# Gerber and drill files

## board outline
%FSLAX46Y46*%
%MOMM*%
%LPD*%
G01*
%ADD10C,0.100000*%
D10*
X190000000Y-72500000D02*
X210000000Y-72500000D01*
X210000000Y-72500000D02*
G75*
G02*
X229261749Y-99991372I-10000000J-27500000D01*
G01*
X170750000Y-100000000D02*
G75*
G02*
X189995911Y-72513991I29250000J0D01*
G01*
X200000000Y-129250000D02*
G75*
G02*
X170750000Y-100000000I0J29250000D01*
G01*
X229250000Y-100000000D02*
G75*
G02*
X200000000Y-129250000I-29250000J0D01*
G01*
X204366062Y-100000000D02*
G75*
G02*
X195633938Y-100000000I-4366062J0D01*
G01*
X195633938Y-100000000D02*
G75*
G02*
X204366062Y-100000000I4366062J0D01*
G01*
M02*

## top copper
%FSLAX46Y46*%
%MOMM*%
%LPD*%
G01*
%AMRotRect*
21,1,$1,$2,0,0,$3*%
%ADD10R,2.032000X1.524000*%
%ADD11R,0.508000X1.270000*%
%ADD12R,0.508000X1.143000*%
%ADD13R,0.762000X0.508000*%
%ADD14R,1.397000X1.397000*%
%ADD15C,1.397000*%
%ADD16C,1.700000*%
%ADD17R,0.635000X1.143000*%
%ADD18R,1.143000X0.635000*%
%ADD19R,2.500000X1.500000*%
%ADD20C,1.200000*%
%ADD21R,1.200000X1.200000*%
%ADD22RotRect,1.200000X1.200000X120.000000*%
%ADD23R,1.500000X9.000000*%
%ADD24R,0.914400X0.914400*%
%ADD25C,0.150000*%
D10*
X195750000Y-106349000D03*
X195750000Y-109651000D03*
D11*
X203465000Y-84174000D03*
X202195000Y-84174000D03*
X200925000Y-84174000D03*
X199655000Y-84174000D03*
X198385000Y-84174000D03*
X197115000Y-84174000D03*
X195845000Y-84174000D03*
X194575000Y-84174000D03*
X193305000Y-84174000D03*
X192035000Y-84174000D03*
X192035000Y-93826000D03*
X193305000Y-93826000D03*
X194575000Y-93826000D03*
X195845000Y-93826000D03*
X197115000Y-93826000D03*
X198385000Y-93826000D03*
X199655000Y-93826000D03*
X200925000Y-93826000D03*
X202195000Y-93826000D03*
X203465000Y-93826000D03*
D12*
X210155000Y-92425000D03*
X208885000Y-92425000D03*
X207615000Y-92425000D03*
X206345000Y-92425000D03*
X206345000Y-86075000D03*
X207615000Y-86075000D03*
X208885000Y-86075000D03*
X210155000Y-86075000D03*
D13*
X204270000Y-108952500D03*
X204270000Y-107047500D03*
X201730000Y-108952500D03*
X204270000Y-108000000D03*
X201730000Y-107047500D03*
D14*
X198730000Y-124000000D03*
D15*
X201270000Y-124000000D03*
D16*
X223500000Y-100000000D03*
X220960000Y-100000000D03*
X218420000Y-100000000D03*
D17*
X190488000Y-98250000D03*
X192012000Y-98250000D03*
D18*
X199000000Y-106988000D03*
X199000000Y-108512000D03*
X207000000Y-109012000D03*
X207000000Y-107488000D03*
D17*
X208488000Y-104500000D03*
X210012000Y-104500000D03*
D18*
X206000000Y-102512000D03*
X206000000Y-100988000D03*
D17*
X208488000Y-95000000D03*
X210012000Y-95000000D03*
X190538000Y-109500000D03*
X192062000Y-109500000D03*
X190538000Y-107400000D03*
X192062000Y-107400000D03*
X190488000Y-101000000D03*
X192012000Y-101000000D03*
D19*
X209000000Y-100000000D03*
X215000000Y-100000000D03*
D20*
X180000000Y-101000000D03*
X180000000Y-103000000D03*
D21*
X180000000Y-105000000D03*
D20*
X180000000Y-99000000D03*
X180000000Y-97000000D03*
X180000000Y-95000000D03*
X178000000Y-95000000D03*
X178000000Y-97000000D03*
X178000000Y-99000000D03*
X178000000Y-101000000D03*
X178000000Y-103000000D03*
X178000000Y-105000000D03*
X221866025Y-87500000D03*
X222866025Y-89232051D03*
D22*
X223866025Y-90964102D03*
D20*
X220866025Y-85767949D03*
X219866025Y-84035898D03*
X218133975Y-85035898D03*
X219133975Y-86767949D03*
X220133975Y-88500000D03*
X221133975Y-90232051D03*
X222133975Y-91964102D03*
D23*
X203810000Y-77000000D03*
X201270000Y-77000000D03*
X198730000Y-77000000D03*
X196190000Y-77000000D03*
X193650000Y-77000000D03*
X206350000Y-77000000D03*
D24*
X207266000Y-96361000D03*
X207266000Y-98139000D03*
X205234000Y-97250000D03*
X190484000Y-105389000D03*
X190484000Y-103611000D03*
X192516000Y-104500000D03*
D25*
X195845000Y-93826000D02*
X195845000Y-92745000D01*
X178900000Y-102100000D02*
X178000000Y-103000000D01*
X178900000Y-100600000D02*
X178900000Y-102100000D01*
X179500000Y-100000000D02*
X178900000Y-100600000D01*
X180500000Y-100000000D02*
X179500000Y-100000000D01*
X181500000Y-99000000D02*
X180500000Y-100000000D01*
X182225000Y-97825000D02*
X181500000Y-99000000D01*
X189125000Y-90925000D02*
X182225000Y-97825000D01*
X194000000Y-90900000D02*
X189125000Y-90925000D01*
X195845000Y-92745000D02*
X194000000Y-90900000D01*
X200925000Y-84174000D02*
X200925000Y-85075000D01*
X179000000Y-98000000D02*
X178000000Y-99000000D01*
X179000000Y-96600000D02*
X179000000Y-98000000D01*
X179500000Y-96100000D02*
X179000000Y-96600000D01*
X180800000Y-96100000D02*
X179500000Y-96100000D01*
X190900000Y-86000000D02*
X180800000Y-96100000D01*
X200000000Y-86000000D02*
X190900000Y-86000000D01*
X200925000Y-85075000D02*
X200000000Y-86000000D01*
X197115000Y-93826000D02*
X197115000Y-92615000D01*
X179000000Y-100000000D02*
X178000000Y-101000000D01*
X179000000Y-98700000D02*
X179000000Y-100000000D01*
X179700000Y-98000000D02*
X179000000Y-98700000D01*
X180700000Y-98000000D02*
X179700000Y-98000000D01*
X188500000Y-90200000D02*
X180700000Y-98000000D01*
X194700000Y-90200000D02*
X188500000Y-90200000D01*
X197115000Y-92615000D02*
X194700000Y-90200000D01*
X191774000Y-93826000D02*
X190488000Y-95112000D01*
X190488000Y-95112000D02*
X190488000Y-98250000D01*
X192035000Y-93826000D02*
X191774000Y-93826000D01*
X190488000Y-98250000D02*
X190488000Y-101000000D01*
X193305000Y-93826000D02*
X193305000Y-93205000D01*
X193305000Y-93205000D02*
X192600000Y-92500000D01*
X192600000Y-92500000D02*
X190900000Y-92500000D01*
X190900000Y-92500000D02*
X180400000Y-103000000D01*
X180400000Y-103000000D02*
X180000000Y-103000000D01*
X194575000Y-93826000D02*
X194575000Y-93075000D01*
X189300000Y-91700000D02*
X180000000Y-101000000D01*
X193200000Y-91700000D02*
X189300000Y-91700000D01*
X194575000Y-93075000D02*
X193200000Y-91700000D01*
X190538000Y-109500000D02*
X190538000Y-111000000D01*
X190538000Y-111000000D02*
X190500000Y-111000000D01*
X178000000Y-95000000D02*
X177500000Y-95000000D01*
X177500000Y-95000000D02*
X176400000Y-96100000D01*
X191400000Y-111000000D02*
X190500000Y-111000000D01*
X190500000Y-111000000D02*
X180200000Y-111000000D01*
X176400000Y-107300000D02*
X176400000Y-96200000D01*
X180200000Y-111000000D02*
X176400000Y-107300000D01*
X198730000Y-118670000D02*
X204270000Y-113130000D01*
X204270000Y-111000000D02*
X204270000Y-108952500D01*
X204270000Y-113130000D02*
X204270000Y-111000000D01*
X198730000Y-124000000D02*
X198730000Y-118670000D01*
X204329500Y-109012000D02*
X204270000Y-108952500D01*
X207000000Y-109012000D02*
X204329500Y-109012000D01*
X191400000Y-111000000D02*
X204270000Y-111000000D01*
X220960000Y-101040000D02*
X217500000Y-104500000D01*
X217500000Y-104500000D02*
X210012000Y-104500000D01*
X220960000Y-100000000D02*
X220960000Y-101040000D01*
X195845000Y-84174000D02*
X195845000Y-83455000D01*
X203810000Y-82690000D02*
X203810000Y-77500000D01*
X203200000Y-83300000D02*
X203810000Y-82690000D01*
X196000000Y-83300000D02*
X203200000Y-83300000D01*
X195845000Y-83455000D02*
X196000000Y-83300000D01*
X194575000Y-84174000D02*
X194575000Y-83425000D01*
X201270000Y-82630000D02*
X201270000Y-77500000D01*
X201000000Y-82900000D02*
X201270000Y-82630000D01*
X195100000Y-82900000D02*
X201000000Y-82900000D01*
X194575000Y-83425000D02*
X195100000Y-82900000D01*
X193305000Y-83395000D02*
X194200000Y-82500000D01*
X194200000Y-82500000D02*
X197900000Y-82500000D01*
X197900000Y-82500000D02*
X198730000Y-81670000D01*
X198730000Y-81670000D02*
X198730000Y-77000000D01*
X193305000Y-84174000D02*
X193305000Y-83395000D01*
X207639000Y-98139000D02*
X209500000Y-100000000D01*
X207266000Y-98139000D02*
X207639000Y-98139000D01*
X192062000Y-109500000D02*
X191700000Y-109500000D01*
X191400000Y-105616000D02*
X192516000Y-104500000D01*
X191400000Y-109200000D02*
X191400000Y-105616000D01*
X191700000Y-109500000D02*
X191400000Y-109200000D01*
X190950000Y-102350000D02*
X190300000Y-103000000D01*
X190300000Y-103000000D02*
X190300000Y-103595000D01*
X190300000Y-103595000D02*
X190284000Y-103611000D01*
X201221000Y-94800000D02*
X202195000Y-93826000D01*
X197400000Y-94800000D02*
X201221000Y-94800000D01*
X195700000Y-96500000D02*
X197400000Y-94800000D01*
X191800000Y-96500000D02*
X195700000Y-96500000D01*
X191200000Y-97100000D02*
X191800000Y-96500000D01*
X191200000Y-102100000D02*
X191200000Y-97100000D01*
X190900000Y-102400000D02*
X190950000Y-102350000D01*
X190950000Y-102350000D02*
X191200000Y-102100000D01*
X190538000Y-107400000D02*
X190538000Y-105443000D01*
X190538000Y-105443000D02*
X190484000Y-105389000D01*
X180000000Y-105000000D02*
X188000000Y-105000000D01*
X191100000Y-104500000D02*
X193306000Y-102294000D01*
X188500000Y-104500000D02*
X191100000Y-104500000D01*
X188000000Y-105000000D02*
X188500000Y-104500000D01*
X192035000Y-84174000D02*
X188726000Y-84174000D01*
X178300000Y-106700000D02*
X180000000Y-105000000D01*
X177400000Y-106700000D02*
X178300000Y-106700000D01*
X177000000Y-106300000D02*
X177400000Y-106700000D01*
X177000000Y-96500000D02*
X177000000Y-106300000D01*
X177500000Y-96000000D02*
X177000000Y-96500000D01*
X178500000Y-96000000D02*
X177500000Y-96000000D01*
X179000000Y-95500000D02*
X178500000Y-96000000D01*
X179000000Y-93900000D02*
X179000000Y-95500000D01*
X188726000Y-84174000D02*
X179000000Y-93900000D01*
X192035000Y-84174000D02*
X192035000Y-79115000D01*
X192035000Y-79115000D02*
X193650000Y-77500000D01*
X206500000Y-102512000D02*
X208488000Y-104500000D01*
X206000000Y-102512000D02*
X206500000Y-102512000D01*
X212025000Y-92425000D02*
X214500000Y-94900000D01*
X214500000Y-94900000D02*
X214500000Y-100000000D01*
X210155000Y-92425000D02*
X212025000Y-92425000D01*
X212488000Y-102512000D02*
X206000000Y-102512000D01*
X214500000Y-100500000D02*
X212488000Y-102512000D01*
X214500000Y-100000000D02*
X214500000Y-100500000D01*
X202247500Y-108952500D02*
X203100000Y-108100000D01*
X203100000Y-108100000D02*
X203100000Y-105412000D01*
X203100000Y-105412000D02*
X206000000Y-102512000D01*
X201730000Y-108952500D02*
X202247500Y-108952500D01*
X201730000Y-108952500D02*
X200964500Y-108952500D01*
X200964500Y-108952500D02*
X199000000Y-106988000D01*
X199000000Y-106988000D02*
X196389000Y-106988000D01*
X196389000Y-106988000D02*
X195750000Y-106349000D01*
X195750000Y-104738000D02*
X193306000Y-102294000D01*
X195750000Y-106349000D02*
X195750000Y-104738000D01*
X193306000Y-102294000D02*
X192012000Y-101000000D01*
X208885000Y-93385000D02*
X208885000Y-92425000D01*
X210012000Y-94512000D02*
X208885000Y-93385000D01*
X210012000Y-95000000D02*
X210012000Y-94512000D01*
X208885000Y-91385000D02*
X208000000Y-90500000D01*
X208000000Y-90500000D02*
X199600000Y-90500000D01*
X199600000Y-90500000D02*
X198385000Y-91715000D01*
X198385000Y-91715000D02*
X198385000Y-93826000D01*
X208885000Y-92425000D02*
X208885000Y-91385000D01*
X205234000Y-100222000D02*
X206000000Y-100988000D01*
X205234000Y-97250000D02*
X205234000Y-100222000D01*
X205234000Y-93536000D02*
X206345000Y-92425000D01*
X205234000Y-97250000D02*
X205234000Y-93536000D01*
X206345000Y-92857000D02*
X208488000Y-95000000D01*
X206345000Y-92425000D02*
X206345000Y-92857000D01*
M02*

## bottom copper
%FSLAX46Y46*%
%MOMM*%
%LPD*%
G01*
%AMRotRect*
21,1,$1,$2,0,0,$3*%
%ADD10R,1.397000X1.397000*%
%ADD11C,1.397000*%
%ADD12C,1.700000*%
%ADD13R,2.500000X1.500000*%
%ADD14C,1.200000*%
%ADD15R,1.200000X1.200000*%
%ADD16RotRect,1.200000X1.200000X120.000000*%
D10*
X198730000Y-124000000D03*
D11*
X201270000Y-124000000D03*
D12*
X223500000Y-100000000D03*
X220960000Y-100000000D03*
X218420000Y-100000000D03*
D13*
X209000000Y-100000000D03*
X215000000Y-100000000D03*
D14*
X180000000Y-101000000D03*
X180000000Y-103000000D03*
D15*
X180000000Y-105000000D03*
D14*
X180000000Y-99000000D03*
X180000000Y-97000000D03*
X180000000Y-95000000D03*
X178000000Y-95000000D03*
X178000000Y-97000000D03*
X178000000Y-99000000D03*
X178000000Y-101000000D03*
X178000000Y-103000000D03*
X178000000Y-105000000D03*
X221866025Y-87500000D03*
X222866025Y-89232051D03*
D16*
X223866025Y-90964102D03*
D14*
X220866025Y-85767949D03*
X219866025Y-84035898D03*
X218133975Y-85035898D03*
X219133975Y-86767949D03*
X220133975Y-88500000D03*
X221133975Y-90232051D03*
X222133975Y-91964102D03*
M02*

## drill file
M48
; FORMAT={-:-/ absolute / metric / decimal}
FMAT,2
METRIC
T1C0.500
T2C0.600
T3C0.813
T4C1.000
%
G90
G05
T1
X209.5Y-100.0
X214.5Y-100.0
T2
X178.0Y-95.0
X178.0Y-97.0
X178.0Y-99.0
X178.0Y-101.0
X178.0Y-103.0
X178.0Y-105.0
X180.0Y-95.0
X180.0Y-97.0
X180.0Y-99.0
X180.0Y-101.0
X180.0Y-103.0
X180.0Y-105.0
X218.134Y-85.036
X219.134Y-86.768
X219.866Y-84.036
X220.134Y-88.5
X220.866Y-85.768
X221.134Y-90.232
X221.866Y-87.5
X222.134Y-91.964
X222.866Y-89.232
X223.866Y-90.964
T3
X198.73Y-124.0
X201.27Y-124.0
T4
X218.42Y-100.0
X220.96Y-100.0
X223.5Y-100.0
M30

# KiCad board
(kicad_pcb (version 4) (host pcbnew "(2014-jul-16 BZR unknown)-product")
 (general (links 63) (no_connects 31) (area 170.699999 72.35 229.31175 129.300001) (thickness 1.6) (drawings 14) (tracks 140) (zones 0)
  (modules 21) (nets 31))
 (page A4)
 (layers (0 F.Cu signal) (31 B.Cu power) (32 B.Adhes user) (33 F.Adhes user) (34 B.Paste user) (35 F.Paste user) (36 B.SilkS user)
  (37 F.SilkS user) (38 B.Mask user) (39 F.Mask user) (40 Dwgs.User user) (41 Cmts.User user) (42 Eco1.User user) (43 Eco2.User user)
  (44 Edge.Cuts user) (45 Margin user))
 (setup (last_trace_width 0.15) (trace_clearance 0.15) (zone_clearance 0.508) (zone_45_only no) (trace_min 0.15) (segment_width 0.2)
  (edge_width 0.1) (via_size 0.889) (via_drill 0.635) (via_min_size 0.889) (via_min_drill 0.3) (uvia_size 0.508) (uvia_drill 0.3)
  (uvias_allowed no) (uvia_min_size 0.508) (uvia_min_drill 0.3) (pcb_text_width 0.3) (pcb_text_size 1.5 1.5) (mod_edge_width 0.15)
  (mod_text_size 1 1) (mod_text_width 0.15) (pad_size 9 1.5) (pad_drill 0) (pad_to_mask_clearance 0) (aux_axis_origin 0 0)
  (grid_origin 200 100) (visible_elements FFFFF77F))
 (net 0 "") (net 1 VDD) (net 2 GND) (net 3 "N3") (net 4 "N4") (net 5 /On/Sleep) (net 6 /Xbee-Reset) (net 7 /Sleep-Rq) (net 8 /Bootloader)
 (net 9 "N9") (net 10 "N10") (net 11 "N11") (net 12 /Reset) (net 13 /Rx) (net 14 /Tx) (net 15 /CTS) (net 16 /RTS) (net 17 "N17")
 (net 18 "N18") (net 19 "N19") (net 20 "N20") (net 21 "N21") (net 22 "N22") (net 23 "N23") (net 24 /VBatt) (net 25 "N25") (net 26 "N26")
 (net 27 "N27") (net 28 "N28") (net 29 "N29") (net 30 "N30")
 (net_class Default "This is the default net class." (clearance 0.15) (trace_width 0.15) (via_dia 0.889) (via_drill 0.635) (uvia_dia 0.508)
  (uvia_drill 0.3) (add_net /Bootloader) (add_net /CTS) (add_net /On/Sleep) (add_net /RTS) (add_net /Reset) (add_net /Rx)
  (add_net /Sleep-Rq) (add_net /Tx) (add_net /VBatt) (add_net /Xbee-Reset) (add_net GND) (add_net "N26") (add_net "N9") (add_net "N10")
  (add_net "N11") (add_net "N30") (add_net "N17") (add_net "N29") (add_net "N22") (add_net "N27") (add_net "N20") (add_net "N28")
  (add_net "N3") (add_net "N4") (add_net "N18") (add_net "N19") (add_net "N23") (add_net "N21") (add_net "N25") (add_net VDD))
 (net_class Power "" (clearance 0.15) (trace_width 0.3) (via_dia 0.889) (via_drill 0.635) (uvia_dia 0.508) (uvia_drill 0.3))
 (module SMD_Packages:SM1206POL (layer F.Cu) (at 195.75 108 270)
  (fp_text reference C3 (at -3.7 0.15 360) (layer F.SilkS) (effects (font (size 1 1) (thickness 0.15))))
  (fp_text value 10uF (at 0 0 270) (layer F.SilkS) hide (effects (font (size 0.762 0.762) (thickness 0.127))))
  (pad 1 smd rect (at -1.651 0 270) (size 1.524 2.032) (layers F.Cu F.Paste F.Mask) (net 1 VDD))
  (pad 2 smd rect (at 1.651 0 270) (size 1.524 2.032) (layers F.Cu F.Paste F.Mask) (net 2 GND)))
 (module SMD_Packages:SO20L (layer F.Cu) (at 197.75 89)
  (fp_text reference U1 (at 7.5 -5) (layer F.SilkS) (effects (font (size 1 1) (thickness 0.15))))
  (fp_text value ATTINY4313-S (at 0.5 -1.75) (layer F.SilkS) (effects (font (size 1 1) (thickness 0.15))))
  (pad 11 smd rect (at 5.715 -4.826) (size 0.508 1.27) (layers F.Cu F.Paste F.Mask) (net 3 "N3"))
  (pad 12 smd rect (at 4.445 -4.826) (size 0.508 1.27) (layers F.Cu F.Paste F.Mask) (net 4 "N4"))
  (pad 13 smd rect (at 3.175 -4.826) (size 0.508 1.27) (layers F.Cu F.Paste F.Mask) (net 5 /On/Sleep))
  (pad 14 smd rect (at 1.905 -4.826) (size 0.508 1.27) (layers F.Cu F.Paste F.Mask) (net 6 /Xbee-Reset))
  (pad 15 smd rect (at 0.635 -4.826) (size 0.508 1.27) (layers F.Cu F.Paste F.Mask) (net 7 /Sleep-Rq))
  (pad 16 smd rect (at -0.635 -4.826) (size 0.508 1.27) (layers F.Cu F.Paste F.Mask) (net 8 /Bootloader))
  (pad 17 smd rect (at -1.905 -4.826) (size 0.508 1.27) (layers F.Cu F.Paste F.Mask) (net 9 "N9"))
  (pad 18 smd rect (at -3.175 -4.826) (size 0.508 1.27) (layers F.Cu F.Paste F.Mask) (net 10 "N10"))
  (pad 19 smd rect (at -4.445 -4.826) (size 0.508 1.27) (layers F.Cu F.Paste F.Mask) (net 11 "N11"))
  (pad 20 smd rect (at -5.715 -4.826) (size 0.508 1.27) (layers F.Cu F.Paste F.Mask) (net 1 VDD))
  (pad 1 smd rect (at -5.715 4.826) (size 0.508 1.27) (layers F.Cu F.Paste F.Mask) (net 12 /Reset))
  (pad 2 smd rect (at -4.445 4.826) (size 0.508 1.27) (layers F.Cu F.Paste F.Mask) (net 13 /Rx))
  (pad 3 smd rect (at -3.175 4.826) (size 0.508 1.27) (layers F.Cu F.Paste F.Mask) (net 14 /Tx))
  (pad 4 smd rect (at -1.905 4.826) (size 0.508 1.27) (layers F.Cu F.Paste F.Mask) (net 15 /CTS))
  (pad 5 smd rect (at -0.635 4.826) (size 0.508 1.27) (layers F.Cu F.Paste F.Mask) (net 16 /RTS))
  (pad 6 smd rect (at 0.635 4.826) (size 0.508 1.27) (layers F.Cu F.Paste F.Mask) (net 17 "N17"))
  (pad 7 smd rect (at 1.905 4.826) (size 0.508 1.27) (layers F.Cu F.Paste F.Mask) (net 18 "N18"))
  (pad 8 smd rect (at 3.175 4.826) (size 0.508 1.27) (layers F.Cu F.Paste F.Mask) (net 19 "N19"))
  (pad 9 smd rect (at 4.445 4.826) (size 0.508 1.27) (layers F.Cu F.Paste F.Mask) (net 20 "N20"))
  (pad 10 smd rect (at 5.715 4.826) (size 0.508 1.27) (layers F.Cu F.Paste F.Mask) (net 2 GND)))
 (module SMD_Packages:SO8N (layer F.Cu) (at 208.25 89.25 180)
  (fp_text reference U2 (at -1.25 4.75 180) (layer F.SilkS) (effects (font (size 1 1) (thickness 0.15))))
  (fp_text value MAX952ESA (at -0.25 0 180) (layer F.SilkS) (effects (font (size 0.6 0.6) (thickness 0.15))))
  (pad 8 smd rect (at -1.905 -3.175 180) (size 0.508 1.143) (layers F.Cu F.Paste F.Mask) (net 1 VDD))
  (pad 7 smd rect (at -0.635 -3.175 180) (size 0.508 1.143) (layers F.Cu F.Paste F.Mask) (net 17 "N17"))
  (pad 6 smd rect (at 0.635 -3.175 180) (size 0.508 1.143) (layers F.Cu F.Paste F.Mask) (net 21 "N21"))
  (pad 5 smd rect (at 1.905 -3.175 180) (size 0.508 1.143) (layers F.Cu F.Paste F.Mask) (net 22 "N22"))
  (pad 4 smd rect (at 1.905 3.175 180) (size 0.508 1.143) (layers F.Cu F.Paste F.Mask) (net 2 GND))
  (pad 3 smd rect (at 0.635 3.175 180) (size 0.508 1.143) (layers F.Cu F.Paste F.Mask) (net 2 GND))
  (pad 2 smd rect (at -0.635 3.175 180) (size 0.508 1.143) (layers F.Cu F.Paste F.Mask) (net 2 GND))
  (pad 1 smd rect (at -1.905 3.175 180) (size 0.508 1.143) (layers F.Cu F.Paste F.Mask) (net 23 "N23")))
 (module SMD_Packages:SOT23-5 (layer F.Cu) (at 203 108 90)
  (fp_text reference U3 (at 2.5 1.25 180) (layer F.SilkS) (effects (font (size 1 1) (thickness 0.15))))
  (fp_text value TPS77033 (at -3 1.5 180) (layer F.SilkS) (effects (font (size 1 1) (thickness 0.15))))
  (pad 1 smd rect (at -0.9525 1.27 90) (size 0.508 0.762) (layers F.Cu F.Paste F.Mask) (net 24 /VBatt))
  (pad 3 smd rect (at 0.9525 1.27 90) (size 0.508 0.762) (layers F.Cu F.Paste F.Mask) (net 2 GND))
  (pad 5 smd rect (at -0.9525 -1.27 90) (size 0.508 0.762) (layers F.Cu F.Paste F.Mask) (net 1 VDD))
  (pad 2 smd rect (at 0 1.27 90) (size 0.508 0.762) (layers F.Cu F.Paste F.Mask) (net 2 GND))
  (pad 4 smd rect (at 0.9525 -1.27 90) (size 0.508 0.762) (layers F.Cu F.Paste F.Mask) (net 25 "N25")))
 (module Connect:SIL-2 (layer F.Cu) (at 200 124)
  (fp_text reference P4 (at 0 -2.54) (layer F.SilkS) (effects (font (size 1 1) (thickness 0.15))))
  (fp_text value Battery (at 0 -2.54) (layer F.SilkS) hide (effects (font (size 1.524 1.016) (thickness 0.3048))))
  (pad 1 thru_hole rect (at -1.27 0) (size 1.397 1.397) (drill 0.8128) (layers *.Cu *.Mask F.SilkS) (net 24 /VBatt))
  (pad 2 thru_hole circle (at 1.27 0) (size 1.397 1.397) (drill 0.8128) (layers *.Cu *.Mask F.SilkS) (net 2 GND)))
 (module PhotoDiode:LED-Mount (layer F.Cu) (at 223.5 100)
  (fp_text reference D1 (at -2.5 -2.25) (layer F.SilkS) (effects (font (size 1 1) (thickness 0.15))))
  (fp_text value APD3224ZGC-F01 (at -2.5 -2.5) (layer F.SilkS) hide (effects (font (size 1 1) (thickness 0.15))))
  (pad 1 thru_hole circle (at 0 0) (size 1.7 1.7) (drill 1) (layers *.Cu *.Mask F.SilkS) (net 2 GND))
  (pad 2 thru_hole circle (at -2.54 0) (size 1.7 1.7) (drill 1) (layers *.Cu *.Mask F.SilkS) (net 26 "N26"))
  (pad 3 thru_hole circle (at -5.08 0) (size 1.7 1.7) (drill 1) (layers *.Cu *.Mask F.SilkS)))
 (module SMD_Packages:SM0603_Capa (layer F.Cu) (at 191.25 98.25)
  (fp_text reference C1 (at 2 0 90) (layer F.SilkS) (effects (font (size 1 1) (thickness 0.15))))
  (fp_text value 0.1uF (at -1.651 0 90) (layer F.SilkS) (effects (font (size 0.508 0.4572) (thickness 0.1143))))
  (pad 1 smd rect (at -0.762 0) (size 0.635 1.143) (layers F.Cu F.Paste F.Mask) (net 12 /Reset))
  (pad 2 smd rect (at 0.762 0) (size 0.635 1.143) (layers F.Cu F.Paste F.Mask) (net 2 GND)))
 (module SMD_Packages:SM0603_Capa (layer F.Cu) (at 199 107.75 270)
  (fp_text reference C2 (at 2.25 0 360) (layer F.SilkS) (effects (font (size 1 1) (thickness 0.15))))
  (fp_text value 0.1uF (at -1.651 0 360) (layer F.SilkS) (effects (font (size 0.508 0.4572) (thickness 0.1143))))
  (pad 1 smd rect (at -0.762 0 270) (size 0.635 1.143) (layers F.Cu F.Paste F.Mask) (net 1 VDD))
  (pad 2 smd rect (at 0.762 0 270) (size 0.635 1.143) (layers F.Cu F.Paste F.Mask) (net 2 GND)))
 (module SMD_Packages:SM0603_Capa (layer F.Cu) (at 207 108.25 90)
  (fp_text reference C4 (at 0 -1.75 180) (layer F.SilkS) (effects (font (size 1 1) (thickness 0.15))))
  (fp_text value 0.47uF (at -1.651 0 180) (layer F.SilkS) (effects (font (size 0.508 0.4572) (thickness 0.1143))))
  (pad 1 smd rect (at -0.762 0 90) (size 0.635 1.143) (layers F.Cu F.Paste F.Mask) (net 24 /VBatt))
  (pad 2 smd rect (at 0.762 0 90) (size 0.635 1.143) (layers F.Cu F.Paste F.Mask) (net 2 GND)))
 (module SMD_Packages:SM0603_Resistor (layer F.Cu) (at 209.25 104.5)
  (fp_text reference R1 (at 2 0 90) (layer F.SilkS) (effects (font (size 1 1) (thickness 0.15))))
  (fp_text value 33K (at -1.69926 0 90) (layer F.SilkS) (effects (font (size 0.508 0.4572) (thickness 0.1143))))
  (pad 1 smd rect (at -0.762 0) (size 0.635 1.143) (layers F.Cu F.Paste F.Mask) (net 1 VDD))
  (pad 2 smd rect (at 0.762 0) (size 0.635 1.143) (layers F.Cu F.Paste F.Mask) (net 26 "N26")))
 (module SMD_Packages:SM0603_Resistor (layer F.Cu) (at 206 101.75 90)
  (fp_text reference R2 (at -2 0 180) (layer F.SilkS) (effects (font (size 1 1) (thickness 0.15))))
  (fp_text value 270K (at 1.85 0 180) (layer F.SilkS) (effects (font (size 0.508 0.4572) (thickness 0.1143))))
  (pad 1 smd rect (at -0.762 0 90) (size 0.635 1.143) (layers F.Cu F.Paste F.Mask) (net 1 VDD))
  (pad 2 smd rect (at 0.762 0 90) (size 0.635 1.143) (layers F.Cu F.Paste F.Mask) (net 22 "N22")))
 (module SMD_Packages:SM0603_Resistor (layer F.Cu) (at 209.25 95)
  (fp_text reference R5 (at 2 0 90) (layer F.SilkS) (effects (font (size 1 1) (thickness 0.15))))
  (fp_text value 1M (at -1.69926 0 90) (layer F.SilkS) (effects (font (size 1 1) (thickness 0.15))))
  (pad 1 smd rect (at -0.762 0) (size 0.635 1.143) (layers F.Cu F.Paste F.Mask) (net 22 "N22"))
  (pad 2 smd rect (at 0.762 0) (size 0.635 1.143) (layers F.Cu F.Paste F.Mask) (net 17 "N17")))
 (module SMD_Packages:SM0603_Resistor (layer F.Cu) (at 191.3 109.5)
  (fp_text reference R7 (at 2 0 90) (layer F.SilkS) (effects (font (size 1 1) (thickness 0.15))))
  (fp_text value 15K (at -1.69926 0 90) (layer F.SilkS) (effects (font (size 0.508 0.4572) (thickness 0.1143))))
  (pad 1 smd rect (at -0.762 0) (size 0.635 1.143) (layers F.Cu F.Paste F.Mask) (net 24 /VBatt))
  (pad 2 smd rect (at 0.762 0) (size 0.635 1.143) (layers F.Cu F.Paste F.Mask) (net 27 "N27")))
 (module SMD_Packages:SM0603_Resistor (layer F.Cu) (at 191.3 107.4)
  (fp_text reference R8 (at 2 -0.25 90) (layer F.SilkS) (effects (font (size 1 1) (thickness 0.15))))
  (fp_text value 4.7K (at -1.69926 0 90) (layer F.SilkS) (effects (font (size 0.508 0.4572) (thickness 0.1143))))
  (pad 1 smd rect (at -0.762 0) (size 0.635 1.143) (layers F.Cu F.Paste F.Mask) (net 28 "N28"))
  (pad 2 smd rect (at 0.762 0) (size 0.635 1.143) (layers F.Cu F.Paste F.Mask) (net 2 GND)))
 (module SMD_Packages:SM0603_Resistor (layer F.Cu) (at 191.25 101)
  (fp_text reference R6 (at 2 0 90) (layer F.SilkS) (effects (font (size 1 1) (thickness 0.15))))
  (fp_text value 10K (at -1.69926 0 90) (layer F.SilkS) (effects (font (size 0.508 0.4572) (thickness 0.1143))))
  (pad 1 smd rect (at -0.762 0) (size 0.635 1.143) (layers F.Cu F.Paste F.Mask) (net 12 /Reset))
  (pad 2 smd rect (at 0.762 0) (size 0.635 1.143) (layers F.Cu F.Paste F.Mask) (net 1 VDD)))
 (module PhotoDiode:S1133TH (layer F.Cu) (at 212 100)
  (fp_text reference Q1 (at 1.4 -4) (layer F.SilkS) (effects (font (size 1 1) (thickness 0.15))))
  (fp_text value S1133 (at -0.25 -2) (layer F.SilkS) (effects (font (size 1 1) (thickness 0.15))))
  (pad 1 thru_hole rect (at -2.5 0) (size 2.5 1.5) (drill 0.5 (offset -0.5 0)) (layers *.Cu *.Mask F.SilkS) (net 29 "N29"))
  (pad 3 thru_hole rect (at 2.5 0) (size 2.5 1.5) (drill 0.5 (offset 0.5 0)) (layers *.Cu *.Mask F.SilkS) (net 1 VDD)))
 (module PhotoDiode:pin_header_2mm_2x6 (layer F.Cu) (at 179 100 90)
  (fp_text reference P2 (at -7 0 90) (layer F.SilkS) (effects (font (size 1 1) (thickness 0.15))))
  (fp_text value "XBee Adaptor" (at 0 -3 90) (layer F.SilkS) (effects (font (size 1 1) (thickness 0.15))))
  (pad 5 thru_hole circle (at -1 1 90) (size 1.2 1.2) (drill 0.6) (layers *.Cu *.Mask F.SilkS) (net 14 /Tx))
  (pad 3 thru_hole circle (at -3 1 90) (size 1.2 1.2) (drill 0.6) (layers *.Cu *.Mask F.SilkS) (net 13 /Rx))
  (pad 1 thru_hole rect (at -5 1 90) (size 1.2 1.2) (drill 0.6) (layers *.Cu *.Mask F.SilkS) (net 1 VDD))
  (pad 7 thru_hole circle (at 1 1 90) (size 1.2 1.2) (drill 0.6) (layers *.Cu *.Mask F.SilkS) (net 8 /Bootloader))
  (pad 9 thru_hole circle (at 3 1 90) (size 1.2 1.2) (drill 0.6) (layers *.Cu *.Mask F.SilkS) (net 12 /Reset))
  (pad 11 thru_hole circle (at 5 1 90) (size 1.2 1.2) (drill 0.6) (layers *.Cu *.Mask F.SilkS) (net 2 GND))
  (pad 12 thru_hole circle (at 5 -1 90) (size 1.2 1.2) (drill 0.6) (layers *.Cu *.Mask F.SilkS) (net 24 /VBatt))
  (pad 10 thru_hole circle (at 3 -1 90) (size 1.2 1.2) (drill 0.6) (layers *.Cu *.Mask F.SilkS) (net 6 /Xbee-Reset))
  (pad 8 thru_hole circle (at 1 -1 90) (size 1.2 1.2) (drill 0.6) (layers *.Cu *.Mask F.SilkS) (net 5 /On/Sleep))
  (pad 6 thru_hole circle (at -1 -1 90) (size 1.2 1.2) (drill 0.6) (layers *.Cu *.Mask F.SilkS) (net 16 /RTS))
  (pad 4 thru_hole circle (at -3 -1 90) (size 1.2 1.2) (drill 0.6) (layers *.Cu *.Mask F.SilkS) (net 15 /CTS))
  (pad 2 thru_hole circle (at -5 -1 90) (size 1.2 1.2) (drill 0.6) (layers *.Cu *.Mask F.SilkS) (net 7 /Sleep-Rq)))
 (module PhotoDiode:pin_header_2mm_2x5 (layer F.Cu) (at 221 88 120)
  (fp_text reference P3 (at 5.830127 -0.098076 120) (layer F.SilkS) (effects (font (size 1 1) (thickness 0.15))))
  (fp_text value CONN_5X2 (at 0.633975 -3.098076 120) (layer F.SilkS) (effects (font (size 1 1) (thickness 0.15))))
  (pad 5 thru_hole circle (at 0 1 120) (size 1.2 1.2) (drill 0.6) (layers *.Cu *.Mask F.SilkS) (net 17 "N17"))
  (pad 3 thru_hole circle (at -2 1 120) (size 1.2 1.2) (drill 0.6) (layers *.Cu *.Mask F.SilkS) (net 14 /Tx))
  (pad 1 thru_hole rect (at -4 1 120) (size 1.2 1.2) (drill 0.6) (layers *.Cu *.Mask F.SilkS) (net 13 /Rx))
  (pad 7 thru_hole circle (at 2 1 120) (size 1.2 1.2) (drill 0.6) (layers *.Cu *.Mask F.SilkS) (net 12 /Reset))
  (pad 9 thru_hole circle (at 4 1 120) (size 1.2 1.2) (drill 0.6) (layers *.Cu *.Mask F.SilkS) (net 2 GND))
  (pad 10 thru_hole circle (at 4 -1 120) (size 1.2 1.2) (drill 0.6) (layers *.Cu *.Mask F.SilkS) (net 24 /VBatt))
  (pad 8 thru_hole circle (at 2 -1 120) (size 1.2 1.2) (drill 0.6) (layers *.Cu *.Mask F.SilkS) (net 6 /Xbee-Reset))
  (pad 6 thru_hole circle (at 0 -1 120) (size 1.2 1.2) (drill 0.6) (layers *.Cu *.Mask F.SilkS) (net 5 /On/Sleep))
  (pad 4 thru_hole circle (at -2 -1 120) (size 1.2 1.2) (drill 0.6) (layers *.Cu *.Mask F.SilkS) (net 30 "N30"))
  (pad 2 thru_hole circle (at -4 -1 120) (size 1.2 1.2) (drill 0.6) (layers *.Cu *.Mask F.SilkS) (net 7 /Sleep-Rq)))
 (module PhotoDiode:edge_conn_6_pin (layer F.Cu) (at 200 77 90)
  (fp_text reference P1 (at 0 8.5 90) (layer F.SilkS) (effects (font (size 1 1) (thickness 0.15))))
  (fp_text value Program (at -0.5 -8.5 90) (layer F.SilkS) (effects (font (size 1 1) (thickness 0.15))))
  (pad 2 connect rect (at 0 3.81 90) (size 9 1.5) (layers F.Cu F.Mask) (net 9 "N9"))
  (pad 3 connect rect (at 0 1.27 90) (size 9 1.5) (layers F.Cu F.Mask) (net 10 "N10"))
  (pad 4 connect rect (at 0 -1.27 90) (size 9 1.5) (layers F.Cu F.Mask) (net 11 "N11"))
  (pad 5 connect rect (at 0 -3.81 90) (size 9 1.5) (layers F.Cu F.Mask) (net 12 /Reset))
  (pad 6 connect rect (at 0 -6.35 90) (size 9 1.5) (layers F.Cu F.Mask) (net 1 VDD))
  (pad 1 connect rect (at 0 6.35 90) (size 9 1.5) (layers F.Cu F.Mask) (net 2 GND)))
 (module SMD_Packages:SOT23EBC (layer F.Cu) (at 206.25 97.25 270)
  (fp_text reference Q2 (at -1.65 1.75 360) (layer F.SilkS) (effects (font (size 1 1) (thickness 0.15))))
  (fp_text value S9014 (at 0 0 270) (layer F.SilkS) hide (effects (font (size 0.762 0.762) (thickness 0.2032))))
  (pad 1 smd rect (at -0.889 -1.016 270) (size 0.9144 0.9144) (layers F.Cu F.Paste F.Mask) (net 2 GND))
  (pad 2 smd rect (at 0.889 -1.016 270) (size 0.9144 0.9144) (layers F.Cu F.Paste F.Mask) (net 29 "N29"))
  (pad 3 smd rect (at 0 1.016 270) (size 0.9144 0.9144) (layers F.Cu F.Paste F.Mask) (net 22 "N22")))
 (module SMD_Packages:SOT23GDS (layer F.Cu) (at 191.5 104.5 90)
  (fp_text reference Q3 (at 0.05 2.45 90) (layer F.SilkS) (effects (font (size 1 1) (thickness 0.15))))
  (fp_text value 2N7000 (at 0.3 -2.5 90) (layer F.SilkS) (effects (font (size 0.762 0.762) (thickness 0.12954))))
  (pad S smd rect (at -0.889 -1.016 90) (size 0.9144 0.9144) (layers F.Cu F.Paste F.Mask) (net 28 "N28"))
  (pad G smd rect (at 0.889 -1.016 90) (size 0.9144 0.9144) (layers F.Cu F.Paste F.Mask) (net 20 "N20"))
  (pad D smd rect (at 0 1.016 90) (size 0.9144 0.9144) (layers F.Cu F.Paste F.Mask) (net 27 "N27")))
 (gr_line (start 190 72.5) (end 210 72.5) (angle 90) (layer Edge.Cuts) (width 0.1))
 (gr_arc (start 200 100) (end 210 72.5) (angle 70) (layer Edge.Cuts) (width 0.1))
 (gr_arc (start 200 100) (end 170.75 100) (angle 70) (layer Edge.Cuts) (width 0.1))
 (gr_arc (start 200 100) (end 200 129.25) (angle 90) (layer Edge.Cuts) (width 0.1))
 (gr_arc (start 200 100) (end 229.25 100) (angle 90) (layer Edge.Cuts) (width 0.1))
 (gr_circle (center 200 100) (end 204.25 101) (layer Edge.Cuts) (width 0.1))
 (segment (start 195.845 93.826) (end 195.845 92.745) (width 0.15) (layer F.Cu) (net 15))
 (segment (start 178.9 102.1) (end 178 103) (width 0.15) (layer F.Cu) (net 15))
 (segment (start 178.9 100.6) (end 178.9 102.1) (width 0.15) (layer F.Cu) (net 15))
 (segment (start 179.5 100) (end 178.9 100.6) (width 0.15) (layer F.Cu) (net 15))
 (segment (start 180.5 100) (end 179.5 100) (width 0.15) (layer F.Cu) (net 15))
 (segment (start 181.5 99) (end 180.5 100) (width 0.15) (layer F.Cu) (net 15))
 (segment (start 182.225 97.825) (end 181.5 99) (width 0.15) (layer F.Cu) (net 15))
 (segment (start 189.125 90.925) (end 182.225 97.825) (width 0.15) (layer F.Cu) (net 15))
 (segment (start 194 90.9) (end 189.125 90.925) (width 0.15) (layer F.Cu) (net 15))
 (segment (start 195.845 92.745) (end 194 90.9) (width 0.15) (layer F.Cu) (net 15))
 (segment (start 200.925 84.174) (end 200.925 85.075) (width 0.15) (layer F.Cu) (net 5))
 (segment (start 179 98) (end 178 99) (width 0.15) (layer F.Cu) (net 5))
 (segment (start 179 96.6) (end 179 98) (width 0.15) (layer F.Cu) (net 5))
 (segment (start 179.5 96.1) (end 179 96.6) (width 0.15) (layer F.Cu) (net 5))
 (segment (start 180.8 96.1) (end 179.5 96.1) (width 0.15) (layer F.Cu) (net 5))
 (segment (start 190.9 86) (end 180.8 96.1) (width 0.15) (layer F.Cu) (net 5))
 (segment (start 200 86) (end 190.9 86) (width 0.15) (layer F.Cu) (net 5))
 (segment (start 200.925 85.075) (end 200 86) (width 0.15) (layer F.Cu) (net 5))
 (segment (start 197.115 93.826) (end 197.115 92.615) (width 0.15) (layer F.Cu) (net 16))
 (segment (start 179 100) (end 178 101) (width 0.15) (layer F.Cu) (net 16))
 (segment (start 179 98.7) (end 179 100) (width 0.15) (layer F.Cu) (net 16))
 (segment (start 179.7 98) (end 179 98.7) (width 0.15) (layer F.Cu) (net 16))
 (segment (start 180.7 98) (end 179.7 98) (width 0.15) (layer F.Cu) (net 16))
 (segment (start 188.5 90.2) (end 180.7 98) (width 0.15) (layer F.Cu) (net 16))
 (segment (start 194.7 90.2) (end 188.5 90.2) (width 0.15) (layer F.Cu) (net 16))
 (segment (start 197.115 92.615) (end 194.7 90.2) (width 0.15) (layer F.Cu) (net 16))
 (segment (start 191.774 93.826) (end 190.488 95.112) (width 0.15) (layer F.Cu) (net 12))
 (segment (start 190.488 95.112) (end 190.488 98.25) (width 0.15) (layer F.Cu) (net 12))
 (segment (start 192.035 93.826) (end 191.774 93.826) (width 0.15) (layer F.Cu) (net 12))
 (segment (start 190.488 98.25) (end 190.488 101) (width 0.15) (layer F.Cu) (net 12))
 (segment (start 193.305 93.826) (end 193.305 93.205) (width 0.15) (layer F.Cu) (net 13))
 (segment (start 193.305 93.205) (end 192.6 92.5) (width 0.15) (layer F.Cu) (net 13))
 (segment (start 192.6 92.5) (end 190.9 92.5) (width 0.15) (layer F.Cu) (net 13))
 (segment (start 190.9 92.5) (end 180.4 103) (width 0.15) (layer F.Cu) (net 13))
 (segment (start 180.4 103) (end 180 103) (width 0.15) (layer F.Cu) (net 13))
 (segment (start 194.575 93.826) (end 194.575 93.075) (width 0.15) (layer F.Cu) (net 14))
 (segment (start 189.3 91.7) (end 180 101) (width 0.15) (layer F.Cu) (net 14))
 (segment (start 193.2 91.7) (end 189.3 91.7) (width 0.15) (layer F.Cu) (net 14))
 (segment (start 194.575 93.075) (end 193.2 91.7) (width 0.15) (layer F.Cu) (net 14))
 (segment (start 190.538 109.5) (end 190.538 111) (width 0.15) (layer F.Cu) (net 24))
 (segment (start 190.538 111) (end 190.5 111) (width 0.15) (layer F.Cu) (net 24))
 (segment (start 178 95) (end 177.5 95) (width 0.15) (layer F.Cu) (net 24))
 (segment (start 177.5 95) (end 176.4 96.1) (width 0.15) (layer F.Cu) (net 24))
 (segment (start 191.4 111) (end 190.5 111) (width 0.15) (layer F.Cu) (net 24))
 (segment (start 190.5 111) (end 180.2 111) (width 0.15) (layer F.Cu) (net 24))
 (segment (start 176.4 107.3) (end 176.4 96.2) (width 0.15) (layer F.Cu) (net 24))
 (segment (start 180.2 111) (end 176.4 107.3) (width 0.15) (layer F.Cu) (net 24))
 (segment (start 198.73 118.67) (end 204.27 113.13) (width 0.15) (layer F.Cu) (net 24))
 (segment (start 204.27 111) (end 204.27 108.9525) (width 0.15) (layer F.Cu) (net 24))
 (segment (start 204.27 113.13) (end 204.27 111) (width 0.15) (layer F.Cu) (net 24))
 (segment (start 198.73 124) (end 198.73 118.67) (width 0.15) (layer F.Cu) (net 24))
 (segment (start 204.3295 109.012) (end 204.27 108.9525) (width 0.15) (layer F.Cu) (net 24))
 (segment (start 207 109.012) (end 204.3295 109.012) (width 0.15) (layer F.Cu) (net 24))
 (segment (start 191.4 111) (end 204.27 111) (width 0.15) (layer F.Cu) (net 24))
 (segment (start 220.96 101.04) (end 217.5 104.5) (width 0.15) (layer F.Cu) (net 26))
 (segment (start 217.5 104.5) (end 210.012 104.5) (width 0.15) (layer F.Cu) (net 26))
 (segment (start 220.96 100) (end 220.96 101.04) (width 0.15) (layer F.Cu) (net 26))
 (segment (start 195.845 84.174) (end 195.845 83.455) (width 0.15) (layer F.Cu) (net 9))
 (segment (start 203.81 82.69) (end 203.81 77.5) (width 0.15) (layer F.Cu) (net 9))
 (segment (start 203.2 83.3) (end 203.81 82.69) (width 0.15) (layer F.Cu) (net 9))
 (segment (start 196 83.3) (end 203.2 83.3) (width 0.15) (layer F.Cu) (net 9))
 (segment (start 195.845 83.455) (end 196 83.3) (width 0.15) (layer F.Cu) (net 9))
 (segment (start 194.575 84.174) (end 194.575 83.425) (width 0.15) (layer F.Cu) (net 10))
 (segment (start 201.27 82.63) (end 201.27 77.5) (width 0.15) (layer F.Cu) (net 10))
 (segment (start 201 82.9) (end 201.27 82.63) (width 0.15) (layer F.Cu) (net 10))
 (segment (start 195.1 82.9) (end 201 82.9) (width 0.15) (layer F.Cu) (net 10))
 (segment (start 194.575 83.425) (end 195.1 82.9) (width 0.15) (layer F.Cu) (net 10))
 (segment (start 193.305 83.395) (end 194.2 82.5) (width 0.15) (layer F.Cu) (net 11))
 (segment (start 194.2 82.5) (end 197.9 82.5) (width 0.15) (layer F.Cu) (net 11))
 (segment (start 197.9 82.5) (end 198.73 81.67) (width 0.15) (layer F.Cu) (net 11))
 (segment (start 198.73 81.67) (end 198.73 77) (width 0.15) (layer F.Cu) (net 11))
 (segment (start 193.305 84.174) (end 193.305 83.395) (width 0.15) (layer F.Cu) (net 11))
 (segment (start 207.639 98.139) (end 209.5 100) (width 0.15) (layer F.Cu) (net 29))
 (segment (start 207.266 98.139) (end 207.639 98.139) (width 0.15) (layer F.Cu) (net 29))
 (segment (start 192.062 109.5) (end 191.7 109.5) (width 0.15) (layer F.Cu) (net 27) (status 400000))
 (segment (start 191.4 105.616) (end 192.516 104.5) (width 0.15) (layer F.Cu) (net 27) (status 800000))
 (segment (start 191.4 109.2) (end 191.4 105.616) (width 0.15) (layer F.Cu) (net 27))
 (segment (start 191.7 109.5) (end 191.4 109.2) (width 0.15) (layer F.Cu) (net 27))
 (segment (start 190.95 102.35) (end 190.3 103) (width 0.15) (layer F.Cu) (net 20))
 (segment (start 190.3 103) (end 190.3 103.595) (width 0.15) (layer F.Cu) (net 20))
 (segment (start 190.3 103.595) (end 190.284 103.611) (width 0.15) (layer F.Cu) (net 20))
 (segment (start 201.221 94.8) (end 202.195 93.826) (width 0.15) (layer F.Cu) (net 20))
 (segment (start 197.4 94.8) (end 201.221 94.8) (width 0.15) (layer F.Cu) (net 20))
 (segment (start 195.7 96.5) (end 197.4 94.8) (width 0.15) (layer F.Cu) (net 20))
 (segment (start 191.8 96.5) (end 195.7 96.5) (width 0.15) (layer F.Cu) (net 20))
 (segment (start 191.2 97.1) (end 191.8 96.5) (width 0.15) (layer F.Cu) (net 20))
 (segment (start 191.2 102.1) (end 191.2 97.1) (width 0.15) (layer F.Cu) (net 20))
 (segment (start 190.9 102.4) (end 190.95 102.35) (width 0.15) (layer F.Cu) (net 20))
 (segment (start 190.95 102.35) (end 191.2 102.1) (width 0.15) (layer F.Cu) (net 20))
 (segment (start 190.538 107.4) (end 190.538 105.443) (width 0.15) (layer F.Cu) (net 28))
 (segment (start 190.538 105.443) (end 190.484 105.389) (width 0.15) (layer F.Cu) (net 28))
 (segment (start 180 105) (end 188 105) (width 0.15) (layer F.Cu) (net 1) (status 400000))
 (segment (start 191.1 104.5) (end 193.306 102.294) (width 0.15) (layer F.Cu) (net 1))
 (segment (start 188.5 104.5) (end 191.1 104.5) (width 0.15) (layer F.Cu) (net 1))
 (segment (start 188 105) (end 188.5 104.5) (width 0.15) (layer F.Cu) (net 1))
 (segment (start 192.035 84.174) (end 188.726 84.174) (width 0.15) (layer F.Cu) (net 1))
 (segment (start 178.3 106.7) (end 180 105) (width 0.15) (layer F.Cu) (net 1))
 (segment (start 177.4 106.7) (end 178.3 106.7) (width 0.15) (layer F.Cu) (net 1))
 (segment (start 177 106.3) (end 177.4 106.7) (width 0.15) (layer F.Cu) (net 1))
 (segment (start 177 96.5) (end 177 106.3) (width 0.15) (layer F.Cu) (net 1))
 (segment (start 177.5 96) (end 177 96.5) (width 0.15) (layer F.Cu) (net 1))
 (segment (start 178.5 96) (end 177.5 96) (width 0.15) (layer F.Cu) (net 1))
 (segment (start 179 95.5) (end 178.5 96) (width 0.15) (layer F.Cu) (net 1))
 (segment (start 179 93.9) (end 179 95.5) (width 0.15) (layer F.Cu) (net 1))
 (segment (start 188.726 84.174) (end 179 93.9) (width 0.15) (layer F.Cu) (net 1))
 (segment (start 192.035 84.174) (end 192.035 79.115) (width 0.15) (layer F.Cu) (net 1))
 (segment (start 192.035 79.115) (end 193.65 77.5) (width 0.15) (layer F.Cu) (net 1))
 (segment (start 206.5 102.512) (end 208.488 104.5) (width 0.15) (layer F.Cu) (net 1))
 (segment (start 206 102.512) (end 206.5 102.512) (width 0.15) (layer F.Cu) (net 1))
 (segment (start 212.025 92.425) (end 214.5 94.9) (width 0.15) (layer F.Cu) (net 1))
 (segment (start 214.5 94.9) (end 214.5 100) (width 0.15) (layer F.Cu) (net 1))
 (segment (start 210.155 92.425) (end 212.025 92.425) (width 0.15) (layer F.Cu) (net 1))
 (segment (start 212.488 102.512) (end 206 102.512) (width 0.15) (layer F.Cu) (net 1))
 (segment (start 214.5 100.5) (end 212.488 102.512) (width 0.15) (layer F.Cu) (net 1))
 (segment (start 214.5 100) (end 214.5 100.5) (width 0.15) (layer F.Cu) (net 1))
 (segment (start 202.2475 108.9525) (end 203.1 108.1) (width 0.15) (layer F.Cu) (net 1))
 (segment (start 203.1 108.1) (end 203.1 105.412) (width 0.15) (layer F.Cu) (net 1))
 (segment (start 203.1 105.412) (end 206 102.512) (width 0.15) (layer F.Cu) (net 1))
 (segment (start 201.73 108.9525) (end 202.2475 108.9525) (width 0.15) (layer F.Cu) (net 1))
 (segment (start 201.73 108.9525) (end 200.9645 108.9525) (width 0.15) (layer F.Cu) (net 1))
 (segment (start 200.9645 108.9525) (end 199 106.988) (width 0.15) (layer F.Cu) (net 1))
 (segment (start 199 106.988) (end 196.389 106.988) (width 0.15) (layer F.Cu) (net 1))
 (segment (start 196.389 106.988) (end 195.75 106.349) (width 0.15) (layer F.Cu) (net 1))
 (segment (start 195.75 104.738) (end 193.306 102.294) (width 0.15) (layer F.Cu) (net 1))
 (segment (start 195.75 106.349) (end 195.75 104.738) (width 0.15) (layer F.Cu) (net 1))
 (segment (start 193.306 102.294) (end 192.012 101) (width 0.15) (layer F.Cu) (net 1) (status 2))
 (segment (start 208.885 93.385) (end 208.885 92.425) (width 0.15) (layer F.Cu) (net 17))
 (segment (start 210.012 94.512) (end 208.885 93.385) (width 0.15) (layer F.Cu) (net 17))
 (segment (start 210.012 95) (end 210.012 94.512) (width 0.15) (layer F.Cu) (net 17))
 (segment (start 208.885 91.385) (end 208 90.5) (width 0.15) (layer F.Cu) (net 17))
 (segment (start 208 90.5) (end 199.6 90.5) (width 0.15) (layer F.Cu) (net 17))
 (segment (start 199.6 90.5) (end 198.385 91.715) (width 0.15) (layer F.Cu) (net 17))
 (segment (start 198.385 91.715) (end 198.385 93.826) (width 0.15) (layer F.Cu) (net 17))
 (segment (start 208.885 92.425) (end 208.885 91.385) (width 0.15) (layer F.Cu) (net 17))
 (segment (start 205.234 100.222) (end 206 100.988) (width 0.15) (layer F.Cu) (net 22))
 (segment (start 205.234 97.25) (end 205.234 100.222) (width 0.15) (layer F.Cu) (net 22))
 (segment (start 205.234 93.536) (end 206.345 92.425) (width 0.15) (layer F.Cu) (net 22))
 (segment (start 205.234 97.25) (end 205.234 93.536) (width 0.15) (layer F.Cu) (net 22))
 (segment (start 206.345 92.857) (end 208.488 95) (width 0.15) (layer F.Cu) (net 22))
 (segment (start 206.345 92.425) (end 206.345 92.857) (width 0.15) (layer F.Cu) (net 22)))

